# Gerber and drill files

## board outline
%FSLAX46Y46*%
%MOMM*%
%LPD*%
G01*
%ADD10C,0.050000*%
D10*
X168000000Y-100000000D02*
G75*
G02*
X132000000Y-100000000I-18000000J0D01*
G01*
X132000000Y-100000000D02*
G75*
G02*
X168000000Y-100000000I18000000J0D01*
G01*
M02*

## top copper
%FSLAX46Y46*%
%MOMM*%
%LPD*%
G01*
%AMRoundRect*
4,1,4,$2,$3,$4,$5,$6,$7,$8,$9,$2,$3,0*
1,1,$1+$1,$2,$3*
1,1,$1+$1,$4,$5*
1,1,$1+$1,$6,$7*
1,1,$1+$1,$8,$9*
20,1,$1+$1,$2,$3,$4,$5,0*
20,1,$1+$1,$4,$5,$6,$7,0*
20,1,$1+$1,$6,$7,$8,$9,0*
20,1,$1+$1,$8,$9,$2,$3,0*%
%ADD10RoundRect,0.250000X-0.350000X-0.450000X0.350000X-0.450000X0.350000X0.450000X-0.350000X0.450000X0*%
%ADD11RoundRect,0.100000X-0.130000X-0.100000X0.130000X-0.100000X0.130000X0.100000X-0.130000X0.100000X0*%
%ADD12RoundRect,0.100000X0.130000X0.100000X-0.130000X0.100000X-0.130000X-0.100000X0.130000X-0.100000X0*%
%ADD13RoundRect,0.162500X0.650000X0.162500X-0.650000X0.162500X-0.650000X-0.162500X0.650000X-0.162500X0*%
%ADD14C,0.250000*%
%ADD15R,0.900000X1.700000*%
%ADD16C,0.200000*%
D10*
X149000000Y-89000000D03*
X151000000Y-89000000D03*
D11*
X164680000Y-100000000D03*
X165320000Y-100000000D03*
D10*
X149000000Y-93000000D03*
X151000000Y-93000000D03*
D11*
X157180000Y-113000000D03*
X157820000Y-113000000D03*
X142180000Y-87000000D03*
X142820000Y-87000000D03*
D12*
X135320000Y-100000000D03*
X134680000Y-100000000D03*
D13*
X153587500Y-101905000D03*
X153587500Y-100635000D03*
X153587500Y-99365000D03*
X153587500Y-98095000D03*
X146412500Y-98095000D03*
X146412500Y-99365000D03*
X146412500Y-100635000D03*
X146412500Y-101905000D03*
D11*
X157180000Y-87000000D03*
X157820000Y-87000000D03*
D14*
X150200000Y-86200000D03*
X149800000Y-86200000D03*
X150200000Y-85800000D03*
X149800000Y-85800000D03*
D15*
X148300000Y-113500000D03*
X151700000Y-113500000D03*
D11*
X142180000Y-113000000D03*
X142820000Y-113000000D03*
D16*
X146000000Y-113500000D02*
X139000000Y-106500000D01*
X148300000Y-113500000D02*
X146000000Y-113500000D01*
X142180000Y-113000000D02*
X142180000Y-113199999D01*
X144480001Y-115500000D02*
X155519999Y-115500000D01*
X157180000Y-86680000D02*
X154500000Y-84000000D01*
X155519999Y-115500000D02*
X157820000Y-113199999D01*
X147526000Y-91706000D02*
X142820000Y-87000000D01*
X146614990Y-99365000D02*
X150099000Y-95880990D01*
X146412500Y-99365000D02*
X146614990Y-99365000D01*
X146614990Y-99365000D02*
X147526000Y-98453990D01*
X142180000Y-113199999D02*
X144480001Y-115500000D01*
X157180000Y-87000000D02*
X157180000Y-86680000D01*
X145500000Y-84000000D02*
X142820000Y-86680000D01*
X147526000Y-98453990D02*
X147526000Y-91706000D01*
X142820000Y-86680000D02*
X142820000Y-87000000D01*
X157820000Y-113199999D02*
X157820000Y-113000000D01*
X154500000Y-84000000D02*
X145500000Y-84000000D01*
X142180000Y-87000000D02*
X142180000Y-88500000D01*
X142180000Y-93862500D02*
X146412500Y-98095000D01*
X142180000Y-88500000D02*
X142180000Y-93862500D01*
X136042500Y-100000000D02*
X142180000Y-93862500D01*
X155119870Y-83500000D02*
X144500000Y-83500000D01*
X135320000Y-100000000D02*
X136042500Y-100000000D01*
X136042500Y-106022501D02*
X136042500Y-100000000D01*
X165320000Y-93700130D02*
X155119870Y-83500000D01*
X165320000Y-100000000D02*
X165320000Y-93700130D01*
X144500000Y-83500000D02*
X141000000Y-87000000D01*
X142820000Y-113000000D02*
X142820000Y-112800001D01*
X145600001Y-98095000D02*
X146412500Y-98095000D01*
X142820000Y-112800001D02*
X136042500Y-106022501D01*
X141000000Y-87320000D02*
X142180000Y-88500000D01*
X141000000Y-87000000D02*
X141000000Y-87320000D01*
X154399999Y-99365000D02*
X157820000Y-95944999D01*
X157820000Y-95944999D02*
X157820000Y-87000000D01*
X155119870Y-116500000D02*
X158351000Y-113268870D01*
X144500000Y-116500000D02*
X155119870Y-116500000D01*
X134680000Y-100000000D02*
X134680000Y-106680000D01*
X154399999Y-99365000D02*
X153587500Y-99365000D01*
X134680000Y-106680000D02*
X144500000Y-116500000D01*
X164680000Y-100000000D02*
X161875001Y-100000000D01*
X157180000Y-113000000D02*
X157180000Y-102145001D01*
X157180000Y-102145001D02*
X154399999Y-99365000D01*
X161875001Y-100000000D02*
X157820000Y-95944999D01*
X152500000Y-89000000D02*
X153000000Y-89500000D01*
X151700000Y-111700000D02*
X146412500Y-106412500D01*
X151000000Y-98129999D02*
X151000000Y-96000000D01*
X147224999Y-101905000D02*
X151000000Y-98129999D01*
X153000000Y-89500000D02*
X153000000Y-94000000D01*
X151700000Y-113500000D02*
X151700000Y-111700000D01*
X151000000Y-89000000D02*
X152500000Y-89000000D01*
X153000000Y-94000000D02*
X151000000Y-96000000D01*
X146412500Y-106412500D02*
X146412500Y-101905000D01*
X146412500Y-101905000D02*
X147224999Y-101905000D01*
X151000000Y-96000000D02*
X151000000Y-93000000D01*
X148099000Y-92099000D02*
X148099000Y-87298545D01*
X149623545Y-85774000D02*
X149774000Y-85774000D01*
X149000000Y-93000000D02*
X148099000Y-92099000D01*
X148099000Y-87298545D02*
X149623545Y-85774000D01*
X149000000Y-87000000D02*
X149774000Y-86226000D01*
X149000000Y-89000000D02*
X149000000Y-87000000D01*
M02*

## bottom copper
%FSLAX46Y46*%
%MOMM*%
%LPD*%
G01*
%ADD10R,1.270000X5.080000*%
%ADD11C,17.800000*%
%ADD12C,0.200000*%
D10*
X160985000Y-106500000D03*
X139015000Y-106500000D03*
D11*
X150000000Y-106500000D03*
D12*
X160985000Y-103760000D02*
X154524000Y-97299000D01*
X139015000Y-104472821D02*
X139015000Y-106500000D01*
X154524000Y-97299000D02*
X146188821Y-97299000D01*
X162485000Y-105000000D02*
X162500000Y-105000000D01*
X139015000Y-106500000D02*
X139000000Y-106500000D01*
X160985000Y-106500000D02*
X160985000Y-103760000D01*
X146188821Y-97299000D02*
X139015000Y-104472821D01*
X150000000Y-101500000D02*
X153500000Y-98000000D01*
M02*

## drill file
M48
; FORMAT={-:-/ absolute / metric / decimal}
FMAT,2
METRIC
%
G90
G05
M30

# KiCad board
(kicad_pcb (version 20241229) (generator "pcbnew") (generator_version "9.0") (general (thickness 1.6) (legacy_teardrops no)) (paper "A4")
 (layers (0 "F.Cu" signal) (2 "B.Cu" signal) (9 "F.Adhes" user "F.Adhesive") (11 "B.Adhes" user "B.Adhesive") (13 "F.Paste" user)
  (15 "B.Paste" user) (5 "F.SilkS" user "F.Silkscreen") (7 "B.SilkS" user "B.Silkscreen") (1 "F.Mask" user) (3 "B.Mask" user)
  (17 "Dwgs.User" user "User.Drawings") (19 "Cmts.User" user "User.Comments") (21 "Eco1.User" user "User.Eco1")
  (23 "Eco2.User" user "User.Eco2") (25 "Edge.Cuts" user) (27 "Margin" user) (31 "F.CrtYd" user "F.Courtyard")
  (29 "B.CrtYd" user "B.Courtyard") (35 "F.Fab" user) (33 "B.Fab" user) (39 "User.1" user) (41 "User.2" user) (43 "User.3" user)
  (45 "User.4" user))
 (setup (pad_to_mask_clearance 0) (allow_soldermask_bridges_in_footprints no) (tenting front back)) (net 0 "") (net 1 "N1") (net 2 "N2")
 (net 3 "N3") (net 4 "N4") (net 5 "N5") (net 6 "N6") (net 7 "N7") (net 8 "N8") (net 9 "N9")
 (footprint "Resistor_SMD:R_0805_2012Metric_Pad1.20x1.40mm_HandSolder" (layer "F.Cu") (at 150 89)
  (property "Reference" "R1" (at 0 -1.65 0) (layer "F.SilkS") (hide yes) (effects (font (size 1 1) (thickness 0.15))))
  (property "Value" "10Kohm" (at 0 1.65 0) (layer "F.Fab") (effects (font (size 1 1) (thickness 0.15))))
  (pad "1" smd roundrect (at -1 0) (size 1.2 1.4) (layers "F.Cu" "F.Mask" "F.Paste") (roundrect_rratio 0.208333) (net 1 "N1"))
  (pad "2" smd roundrect (at 1 0) (size 1.2 1.4) (layers "F.Cu" "F.Mask" "F.Paste") (roundrect_rratio 0.208333) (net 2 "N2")))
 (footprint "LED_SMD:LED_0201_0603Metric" (layer "F.Cu") (at 165 100)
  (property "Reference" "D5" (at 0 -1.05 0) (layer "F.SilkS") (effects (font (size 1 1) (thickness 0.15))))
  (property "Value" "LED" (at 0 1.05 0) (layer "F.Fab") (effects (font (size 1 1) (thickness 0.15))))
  (pad "" smd roundrect (at -0.345 0) (size 0.318 0.36) (layers "F.Paste") (roundrect_rratio 0.25))
  (pad "" smd roundrect (at 0.345 0) (size 0.318 0.36) (layers "F.Paste") (roundrect_rratio 0.25))
  (pad "1" smd roundrect (at -0.32 0) (size 0.46 0.4) (layers "F.Cu" "F.Mask") (roundrect_rratio 0.25) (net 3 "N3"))
  (pad "2" smd roundrect (at 0.32 0) (size 0.46 0.4) (layers "F.Cu" "F.Mask") (roundrect_rratio 0.25) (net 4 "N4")))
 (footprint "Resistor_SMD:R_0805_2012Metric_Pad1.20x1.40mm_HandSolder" (layer "F.Cu") (at 150 93)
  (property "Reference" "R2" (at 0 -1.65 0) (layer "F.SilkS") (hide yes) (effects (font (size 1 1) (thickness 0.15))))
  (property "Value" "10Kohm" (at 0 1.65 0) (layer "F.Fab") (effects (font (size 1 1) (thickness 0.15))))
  (pad "1" smd roundrect (at -1 0) (size 1.2 1.4) (layers "F.Cu" "F.Mask" "F.Paste") (roundrect_rratio 0.208333) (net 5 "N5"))
  (pad "2" smd roundrect (at 1 0) (size 1.2 1.4) (layers "F.Cu" "F.Mask" "F.Paste") (roundrect_rratio 0.208333) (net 2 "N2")))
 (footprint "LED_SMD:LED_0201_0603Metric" (layer "F.Cu") (at 157.5 113)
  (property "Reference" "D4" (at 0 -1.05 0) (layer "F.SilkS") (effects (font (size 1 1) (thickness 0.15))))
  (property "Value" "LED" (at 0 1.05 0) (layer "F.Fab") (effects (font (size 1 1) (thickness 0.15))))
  (pad "" smd roundrect (at -0.345 0) (size 0.318 0.36) (layers "F.Paste") (roundrect_rratio 0.25))
  (pad "" smd roundrect (at 0.345 0) (size 0.318 0.36) (layers "F.Paste") (roundrect_rratio 0.25))
  (pad "1" smd roundrect (at -0.32 0) (size 0.46 0.4) (layers "F.Cu" "F.Mask") (roundrect_rratio 0.25) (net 3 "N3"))
  (pad "2" smd roundrect (at 0.32 0) (size 0.46 0.4) (layers "F.Cu" "F.Mask") (roundrect_rratio 0.25) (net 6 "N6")))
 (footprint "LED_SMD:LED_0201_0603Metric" (layer "F.Cu") (at 142.5 87)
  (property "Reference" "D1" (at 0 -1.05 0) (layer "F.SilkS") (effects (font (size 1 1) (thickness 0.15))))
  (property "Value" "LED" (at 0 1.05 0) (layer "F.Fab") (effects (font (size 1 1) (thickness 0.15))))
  (pad "" smd roundrect (at -0.345 0) (size 0.318 0.36) (layers "F.Paste") (roundrect_rratio 0.25))
  (pad "" smd roundrect (at 0.345 0) (size 0.318 0.36) (layers "F.Paste") (roundrect_rratio 0.25))
  (pad "1" smd roundrect (at -0.32 0) (size 0.46 0.4) (layers "F.Cu" "F.Mask") (roundrect_rratio 0.25) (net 4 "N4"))
  (pad "2" smd roundrect (at 0.32 0) (size 0.46 0.4) (layers "F.Cu" "F.Mask") (roundrect_rratio 0.25) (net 6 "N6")))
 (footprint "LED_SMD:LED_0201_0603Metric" (layer "F.Cu") (at 135 100 180)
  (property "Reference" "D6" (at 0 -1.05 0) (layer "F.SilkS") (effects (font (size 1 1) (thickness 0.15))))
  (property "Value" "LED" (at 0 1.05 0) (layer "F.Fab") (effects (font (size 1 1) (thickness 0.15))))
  (pad "" smd roundrect (at -0.345 0 180) (size 0.318 0.36) (layers "F.Paste") (roundrect_rratio 0.25))
  (pad "" smd roundrect (at 0.345 0 180) (size 0.318 0.36) (layers "F.Paste") (roundrect_rratio 0.25))
  (pad "1" smd roundrect (at -0.32 0 180) (size 0.46 0.4) (layers "F.Cu" "F.Mask") (roundrect_rratio 0.25) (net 4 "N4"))
  (pad "2" smd roundrect (at 0.32 0 180) (size 0.46 0.4) (layers "F.Cu" "F.Mask") (roundrect_rratio 0.25) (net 3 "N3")))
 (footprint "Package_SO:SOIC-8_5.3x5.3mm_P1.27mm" (layer "F.Cu") (at 150 100 180)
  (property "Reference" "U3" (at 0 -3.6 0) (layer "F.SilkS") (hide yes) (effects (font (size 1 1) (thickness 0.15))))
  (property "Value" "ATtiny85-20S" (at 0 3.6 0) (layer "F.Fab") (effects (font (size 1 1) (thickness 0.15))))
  (pad "1" smd roundrect (at -3.5875 -1.905 180) (size 1.625 0.65) (layers "F.Cu" "F.Mask" "F.Paste") (roundrect_rratio 0.25) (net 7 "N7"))
  (pad "2" smd roundrect (at -3.5875 -0.635 180) (size 1.625 0.65) (layers "F.Cu" "F.Mask" "F.Paste") (roundrect_rratio 0.25) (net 5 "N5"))
  (pad "3" smd roundrect (at -3.5875 0.635 180) (size 1.625 0.65) (layers "F.Cu" "F.Mask" "F.Paste") (roundrect_rratio 0.25) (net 3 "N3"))
  (pad "4" smd roundrect (at -3.5875 1.905 180) (size 1.625 0.65) (layers "F.Cu" "F.Mask" "F.Paste") (roundrect_rratio 0.25) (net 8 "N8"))
  (pad "5" smd roundrect (at 3.5875 1.905 180) (size 1.625 0.65) (layers "F.Cu" "F.Mask" "F.Paste") (roundrect_rratio 0.25) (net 4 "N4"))
  (pad "6" smd roundrect (at 3.5875 0.635 180) (size 1.625 0.65) (layers "F.Cu" "F.Mask" "F.Paste") (roundrect_rratio 0.25) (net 6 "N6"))
  (pad "7" smd roundrect (at 3.5875 -0.635 180) (size 1.625 0.65) (layers "F.Cu" "F.Mask" "F.Paste") (roundrect_rratio 0.25) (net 1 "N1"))
  (pad "8" smd roundrect (at 3.5875 -1.905 180) (size 1.625 0.65) (layers "F.Cu" "F.Mask" "F.Paste") (roundrect_rratio 0.25) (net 2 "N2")))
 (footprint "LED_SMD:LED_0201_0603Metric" (layer "F.Cu") (at 157.5 87)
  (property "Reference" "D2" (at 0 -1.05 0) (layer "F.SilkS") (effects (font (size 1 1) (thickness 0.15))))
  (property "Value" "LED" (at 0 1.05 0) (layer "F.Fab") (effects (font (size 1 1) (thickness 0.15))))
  (pad "" smd roundrect (at -0.345 0) (size 0.318 0.36) (layers "F.Paste") (roundrect_rratio 0.25))
  (pad "" smd roundrect (at 0.345 0) (size 0.318 0.36) (layers "F.Paste") (roundrect_rratio 0.25))
  (pad "1" smd roundrect (at -0.32 0) (size 0.46 0.4) (layers "F.Cu" "F.Mask") (roundrect_rratio 0.25) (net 6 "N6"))
  (pad "2" smd roundrect (at 0.32 0) (size 0.46 0.4) (layers "F.Cu" "F.Mask") (roundrect_rratio 0.25) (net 3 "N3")))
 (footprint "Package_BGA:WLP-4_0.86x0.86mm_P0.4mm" (layer "F.Cu") (at 150 86 180)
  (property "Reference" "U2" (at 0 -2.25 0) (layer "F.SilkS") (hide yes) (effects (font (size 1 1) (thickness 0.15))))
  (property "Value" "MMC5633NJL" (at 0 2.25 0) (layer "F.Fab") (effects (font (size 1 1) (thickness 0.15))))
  (pad "A1" smd circle (at -0.2 -0.2 180) (size 0.25 0.25) (layers "F.Cu" "F.Mask" "F.Paste") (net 8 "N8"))
  (pad "A2" smd circle (at 0.2 -0.2 180) (size 0.25 0.25) (layers "F.Cu" "F.Mask" "F.Paste") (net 1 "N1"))
  (pad "B1" smd circle (at -0.2 0.2 180) (size 0.25 0.25) (layers "F.Cu" "F.Mask" "F.Paste") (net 2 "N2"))
  (pad "B2" smd circle (at 0.2 0.2 180) (size 0.25 0.25) (layers "F.Cu" "F.Mask" "F.Paste") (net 5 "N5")))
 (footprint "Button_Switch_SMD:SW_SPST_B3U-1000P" (layer "F.Cu") (at 150 113.5)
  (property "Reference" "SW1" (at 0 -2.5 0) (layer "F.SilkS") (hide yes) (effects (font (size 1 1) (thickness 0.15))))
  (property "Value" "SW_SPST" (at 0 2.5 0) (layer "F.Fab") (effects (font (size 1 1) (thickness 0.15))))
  (pad "1" smd rect (at -1.7 0) (size 0.9 1.7) (layers "F.Cu" "F.Mask" "F.Paste") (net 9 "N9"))
  (pad "2" smd rect (at 1.7 0) (size 0.9 1.7) (layers "F.Cu" "F.Mask" "F.Paste") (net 2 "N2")))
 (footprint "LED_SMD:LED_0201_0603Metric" (layer "F.Cu") (at 142.5 113)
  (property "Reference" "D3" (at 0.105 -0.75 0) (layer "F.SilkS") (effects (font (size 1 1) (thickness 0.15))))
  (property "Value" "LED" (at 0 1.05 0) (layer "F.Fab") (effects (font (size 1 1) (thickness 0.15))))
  (pad "" smd roundrect (at -0.345 0) (size 0.318 0.36) (layers "F.Paste") (roundrect_rratio 0.25))
  (pad "" smd roundrect (at 0.345 0) (size 0.318 0.36) (layers "F.Paste") (roundrect_rratio 0.25))
  (pad "1" smd roundrect (at -0.32 0) (size 0.46 0.4) (layers "F.Cu" "F.Mask") (roundrect_rratio 0.25) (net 6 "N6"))
  (pad "2" smd roundrect (at 0.32 0) (size 0.46 0.4) (layers "F.Cu" "F.Mask") (roundrect_rratio 0.25) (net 4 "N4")))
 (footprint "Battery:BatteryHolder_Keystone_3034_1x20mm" (layer "B.Cu") (at 150 106.5 180)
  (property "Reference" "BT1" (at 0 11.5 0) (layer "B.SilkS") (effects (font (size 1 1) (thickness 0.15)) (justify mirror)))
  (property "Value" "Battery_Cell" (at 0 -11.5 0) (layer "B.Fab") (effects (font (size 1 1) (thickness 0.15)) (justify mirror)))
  (pad "1" smd rect (at -10.985 0 180) (size 1.27 5.08) (layers "B.Cu" "B.Mask" "B.Paste") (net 9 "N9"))
  (pad "1" smd rect (at 10.985 0 180) (size 1.27 5.08) (layers "B.Cu" "B.Mask" "B.Paste") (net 9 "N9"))
  (pad "2" smd circle (at 0 0 180) (size 17.8 17.8) (layers "B.Cu" "B.Mask") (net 8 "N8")))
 (gr_circle (center 150 100) (end 168 100) (stroke (width 0.05) (type solid)) (fill no) (layer "Edge.Cuts"))
 (segment (start 146 113.5) (end 139 106.5) (width 0.2) (layer "F.Cu") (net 9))
 (segment (start 148.3 113.5) (end 146 113.5) (width 0.2) (layer "F.Cu") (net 9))
 (segment (start 160.985 103.76) (end 154.524 97.299) (width 0.2) (layer "B.Cu") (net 9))
 (segment (start 139.015 104.472821) (end 139.015 106.5) (width 0.2) (layer "B.Cu") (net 9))
 (segment (start 154.524 97.299) (end 146.188821 97.299) (width 0.2) (layer "B.Cu") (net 9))
 (segment (start 162.485 105) (end 162.5 105) (width 0.2) (layer "B.Cu") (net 9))
 (segment (start 139.015 106.5) (end 139 106.5) (width 0.2) (layer "B.Cu") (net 9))
 (segment (start 160.985 106.5) (end 160.985 103.76) (width 0.2) (layer "B.Cu") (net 9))
 (segment (start 146.188821 97.299) (end 139.015 104.472821) (width 0.2) (layer "B.Cu") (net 9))
 (segment (start 150 101.5) (end 153.5 98) (width 0.2) (layer "B.Cu") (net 8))
 (segment (start 142.18 113) (end 142.18 113.199999) (width 0.2) (layer "F.Cu") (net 6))
 (segment (start 144.480001 115.5) (end 155.519999 115.5) (width 0.2) (layer "F.Cu") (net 6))
 (segment (start 157.18 86.68) (end 154.5 84) (width 0.2) (layer "F.Cu") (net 6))
 (segment (start 155.519999 115.5) (end 157.82 113.199999) (width 0.2) (layer "F.Cu") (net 6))
 (segment (start 147.526 91.706) (end 142.82 87) (width 0.2) (layer "F.Cu") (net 6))
 (segment (start 146.61499 99.365) (end 150.099 95.88099) (width 0.2) (layer "F.Cu") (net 6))
 (segment (start 146.4125 99.365) (end 146.61499 99.365) (width 0.2) (layer "F.Cu") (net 6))
 (segment (start 146.61499 99.365) (end 147.526 98.45399) (width 0.2) (layer "F.Cu") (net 6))
 (segment (start 142.18 113.199999) (end 144.480001 115.5) (width 0.2) (layer "F.Cu") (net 6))
 (segment (start 157.18 87) (end 157.18 86.68) (width 0.2) (layer "F.Cu") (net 6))
 (segment (start 145.5 84) (end 142.82 86.68) (width 0.2) (layer "F.Cu") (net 6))
 (segment (start 147.526 98.45399) (end 147.526 91.706) (width 0.2) (layer "F.Cu") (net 6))
 (segment (start 142.82 86.68) (end 142.82 87) (width 0.2) (layer "F.Cu") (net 6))
 (segment (start 157.82 113.199999) (end 157.82 113) (width 0.2) (layer "F.Cu") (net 6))
 (segment (start 154.5 84) (end 145.5 84) (width 0.2) (layer "F.Cu") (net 6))
 (segment (start 142.18 87) (end 142.18 88.5) (width 0.2) (layer "F.Cu") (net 4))
 (segment (start 142.18 93.8625) (end 146.4125 98.095) (width 0.2) (layer "F.Cu") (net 4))
 (segment (start 142.18 88.5) (end 142.18 93.8625) (width 0.2) (layer "F.Cu") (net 4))
 (segment (start 136.0425 100) (end 142.18 93.8625) (width 0.2) (layer "F.Cu") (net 4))
 (segment (start 155.11987 83.5) (end 144.5 83.5) (width 0.2) (layer "F.Cu") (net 4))
 (segment (start 135.32 100) (end 136.0425 100) (width 0.2) (layer "F.Cu") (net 4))
 (segment (start 136.0425 106.022501) (end 136.0425 100) (width 0.2) (layer "F.Cu") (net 4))
 (segment (start 165.32 93.70013) (end 155.11987 83.5) (width 0.2) (layer "F.Cu") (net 4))
 (segment (start 165.32 100) (end 165.32 93.70013) (width 0.2) (layer "F.Cu") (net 4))
 (segment (start 144.5 83.5) (end 141 87) (width 0.2) (layer "F.Cu") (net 4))
 (segment (start 142.82 113) (end 142.82 112.800001) (width 0.2) (layer "F.Cu") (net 4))
 (segment (start 145.600001 98.095) (end 146.4125 98.095) (width 0.2) (layer "F.Cu") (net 4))
 (segment (start 142.82 112.800001) (end 136.0425 106.022501) (width 0.2) (layer "F.Cu") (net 4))
 (segment (start 141 87.32) (end 142.18 88.5) (width 0.2) (layer "F.Cu") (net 4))
 (segment (start 141 87) (end 141 87.32) (width 0.2) (layer "F.Cu") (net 4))
 (segment (start 154.399999 99.365) (end 157.82 95.944999) (width 0.2) (layer "F.Cu") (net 3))
 (segment (start 157.82 95.944999) (end 157.82 87) (width 0.2) (layer "F.Cu") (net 3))
 (segment (start 155.11987 116.5) (end 158.351 113.26887) (width 0.2) (layer "F.Cu") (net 3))
 (segment (start 144.5 116.5) (end 155.11987 116.5) (width 0.2) (layer "F.Cu") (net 3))
 (segment (start 134.68 100) (end 134.68 106.68) (width 0.2) (layer "F.Cu") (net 3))
 (segment (start 154.399999 99.365) (end 153.5875 99.365) (width 0.2) (layer "F.Cu") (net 3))
 (segment (start 134.68 106.68) (end 144.5 116.5) (width 0.2) (layer "F.Cu") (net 3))
 (segment (start 164.68 100) (end 161.875001 100) (width 0.2) (layer "F.Cu") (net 3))
 (segment (start 157.18 113) (end 157.18 102.145001) (width 0.2) (layer "F.Cu") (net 3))
 (segment (start 157.18 102.145001) (end 154.399999 99.365) (width 0.2) (layer "F.Cu") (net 3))
 (segment (start 161.875001 100) (end 157.82 95.944999) (width 0.2) (layer "F.Cu") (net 3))
 (segment (start 152.5 89) (end 153 89.5) (width 0.2) (layer "F.Cu") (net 2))
 (segment (start 151.7 111.7) (end 146.4125 106.4125) (width 0.2) (layer "F.Cu") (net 2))
 (segment (start 151 98.129999) (end 151 96) (width 0.2) (layer "F.Cu") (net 2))
 (segment (start 147.224999 101.905) (end 151 98.129999) (width 0.2) (layer "F.Cu") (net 2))
 (segment (start 153 89.5) (end 153 94) (width 0.2) (layer "F.Cu") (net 2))
 (segment (start 151.7 113.5) (end 151.7 111.7) (width 0.2) (layer "F.Cu") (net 2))
 (segment (start 151 89) (end 152.5 89) (width 0.2) (layer "F.Cu") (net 2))
 (segment (start 153 94) (end 151 96) (width 0.2) (layer "F.Cu") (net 2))
 (segment (start 146.4125 106.4125) (end 146.4125 101.905) (width 0.2) (layer "F.Cu") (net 2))
 (segment (start 146.4125 101.905) (end 147.224999 101.905) (width 0.2) (layer "F.Cu") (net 2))
 (segment (start 151 96) (end 151 93) (width 0.2) (layer "F.Cu") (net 2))
 (segment (start 148.099 92.099) (end 148.099 87.298545) (width 0.2) (layer "F.Cu") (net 5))
 (segment (start 149.623545 85.774) (end 149.774 85.774) (width 0.2) (layer "F.Cu") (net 5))
 (segment (start 149 93) (end 148.099 92.099) (width 0.2) (layer "F.Cu") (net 5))
 (segment (start 148.099 87.298545) (end 149.623545 85.774) (width 0.2) (layer "F.Cu") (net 5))
 (segment (start 149 87) (end 149.774 86.226) (width 0.2) (layer "F.Cu") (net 1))
 (segment (start 149 89) (end 149 87) (width 0.2) (layer "F.Cu") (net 1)))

